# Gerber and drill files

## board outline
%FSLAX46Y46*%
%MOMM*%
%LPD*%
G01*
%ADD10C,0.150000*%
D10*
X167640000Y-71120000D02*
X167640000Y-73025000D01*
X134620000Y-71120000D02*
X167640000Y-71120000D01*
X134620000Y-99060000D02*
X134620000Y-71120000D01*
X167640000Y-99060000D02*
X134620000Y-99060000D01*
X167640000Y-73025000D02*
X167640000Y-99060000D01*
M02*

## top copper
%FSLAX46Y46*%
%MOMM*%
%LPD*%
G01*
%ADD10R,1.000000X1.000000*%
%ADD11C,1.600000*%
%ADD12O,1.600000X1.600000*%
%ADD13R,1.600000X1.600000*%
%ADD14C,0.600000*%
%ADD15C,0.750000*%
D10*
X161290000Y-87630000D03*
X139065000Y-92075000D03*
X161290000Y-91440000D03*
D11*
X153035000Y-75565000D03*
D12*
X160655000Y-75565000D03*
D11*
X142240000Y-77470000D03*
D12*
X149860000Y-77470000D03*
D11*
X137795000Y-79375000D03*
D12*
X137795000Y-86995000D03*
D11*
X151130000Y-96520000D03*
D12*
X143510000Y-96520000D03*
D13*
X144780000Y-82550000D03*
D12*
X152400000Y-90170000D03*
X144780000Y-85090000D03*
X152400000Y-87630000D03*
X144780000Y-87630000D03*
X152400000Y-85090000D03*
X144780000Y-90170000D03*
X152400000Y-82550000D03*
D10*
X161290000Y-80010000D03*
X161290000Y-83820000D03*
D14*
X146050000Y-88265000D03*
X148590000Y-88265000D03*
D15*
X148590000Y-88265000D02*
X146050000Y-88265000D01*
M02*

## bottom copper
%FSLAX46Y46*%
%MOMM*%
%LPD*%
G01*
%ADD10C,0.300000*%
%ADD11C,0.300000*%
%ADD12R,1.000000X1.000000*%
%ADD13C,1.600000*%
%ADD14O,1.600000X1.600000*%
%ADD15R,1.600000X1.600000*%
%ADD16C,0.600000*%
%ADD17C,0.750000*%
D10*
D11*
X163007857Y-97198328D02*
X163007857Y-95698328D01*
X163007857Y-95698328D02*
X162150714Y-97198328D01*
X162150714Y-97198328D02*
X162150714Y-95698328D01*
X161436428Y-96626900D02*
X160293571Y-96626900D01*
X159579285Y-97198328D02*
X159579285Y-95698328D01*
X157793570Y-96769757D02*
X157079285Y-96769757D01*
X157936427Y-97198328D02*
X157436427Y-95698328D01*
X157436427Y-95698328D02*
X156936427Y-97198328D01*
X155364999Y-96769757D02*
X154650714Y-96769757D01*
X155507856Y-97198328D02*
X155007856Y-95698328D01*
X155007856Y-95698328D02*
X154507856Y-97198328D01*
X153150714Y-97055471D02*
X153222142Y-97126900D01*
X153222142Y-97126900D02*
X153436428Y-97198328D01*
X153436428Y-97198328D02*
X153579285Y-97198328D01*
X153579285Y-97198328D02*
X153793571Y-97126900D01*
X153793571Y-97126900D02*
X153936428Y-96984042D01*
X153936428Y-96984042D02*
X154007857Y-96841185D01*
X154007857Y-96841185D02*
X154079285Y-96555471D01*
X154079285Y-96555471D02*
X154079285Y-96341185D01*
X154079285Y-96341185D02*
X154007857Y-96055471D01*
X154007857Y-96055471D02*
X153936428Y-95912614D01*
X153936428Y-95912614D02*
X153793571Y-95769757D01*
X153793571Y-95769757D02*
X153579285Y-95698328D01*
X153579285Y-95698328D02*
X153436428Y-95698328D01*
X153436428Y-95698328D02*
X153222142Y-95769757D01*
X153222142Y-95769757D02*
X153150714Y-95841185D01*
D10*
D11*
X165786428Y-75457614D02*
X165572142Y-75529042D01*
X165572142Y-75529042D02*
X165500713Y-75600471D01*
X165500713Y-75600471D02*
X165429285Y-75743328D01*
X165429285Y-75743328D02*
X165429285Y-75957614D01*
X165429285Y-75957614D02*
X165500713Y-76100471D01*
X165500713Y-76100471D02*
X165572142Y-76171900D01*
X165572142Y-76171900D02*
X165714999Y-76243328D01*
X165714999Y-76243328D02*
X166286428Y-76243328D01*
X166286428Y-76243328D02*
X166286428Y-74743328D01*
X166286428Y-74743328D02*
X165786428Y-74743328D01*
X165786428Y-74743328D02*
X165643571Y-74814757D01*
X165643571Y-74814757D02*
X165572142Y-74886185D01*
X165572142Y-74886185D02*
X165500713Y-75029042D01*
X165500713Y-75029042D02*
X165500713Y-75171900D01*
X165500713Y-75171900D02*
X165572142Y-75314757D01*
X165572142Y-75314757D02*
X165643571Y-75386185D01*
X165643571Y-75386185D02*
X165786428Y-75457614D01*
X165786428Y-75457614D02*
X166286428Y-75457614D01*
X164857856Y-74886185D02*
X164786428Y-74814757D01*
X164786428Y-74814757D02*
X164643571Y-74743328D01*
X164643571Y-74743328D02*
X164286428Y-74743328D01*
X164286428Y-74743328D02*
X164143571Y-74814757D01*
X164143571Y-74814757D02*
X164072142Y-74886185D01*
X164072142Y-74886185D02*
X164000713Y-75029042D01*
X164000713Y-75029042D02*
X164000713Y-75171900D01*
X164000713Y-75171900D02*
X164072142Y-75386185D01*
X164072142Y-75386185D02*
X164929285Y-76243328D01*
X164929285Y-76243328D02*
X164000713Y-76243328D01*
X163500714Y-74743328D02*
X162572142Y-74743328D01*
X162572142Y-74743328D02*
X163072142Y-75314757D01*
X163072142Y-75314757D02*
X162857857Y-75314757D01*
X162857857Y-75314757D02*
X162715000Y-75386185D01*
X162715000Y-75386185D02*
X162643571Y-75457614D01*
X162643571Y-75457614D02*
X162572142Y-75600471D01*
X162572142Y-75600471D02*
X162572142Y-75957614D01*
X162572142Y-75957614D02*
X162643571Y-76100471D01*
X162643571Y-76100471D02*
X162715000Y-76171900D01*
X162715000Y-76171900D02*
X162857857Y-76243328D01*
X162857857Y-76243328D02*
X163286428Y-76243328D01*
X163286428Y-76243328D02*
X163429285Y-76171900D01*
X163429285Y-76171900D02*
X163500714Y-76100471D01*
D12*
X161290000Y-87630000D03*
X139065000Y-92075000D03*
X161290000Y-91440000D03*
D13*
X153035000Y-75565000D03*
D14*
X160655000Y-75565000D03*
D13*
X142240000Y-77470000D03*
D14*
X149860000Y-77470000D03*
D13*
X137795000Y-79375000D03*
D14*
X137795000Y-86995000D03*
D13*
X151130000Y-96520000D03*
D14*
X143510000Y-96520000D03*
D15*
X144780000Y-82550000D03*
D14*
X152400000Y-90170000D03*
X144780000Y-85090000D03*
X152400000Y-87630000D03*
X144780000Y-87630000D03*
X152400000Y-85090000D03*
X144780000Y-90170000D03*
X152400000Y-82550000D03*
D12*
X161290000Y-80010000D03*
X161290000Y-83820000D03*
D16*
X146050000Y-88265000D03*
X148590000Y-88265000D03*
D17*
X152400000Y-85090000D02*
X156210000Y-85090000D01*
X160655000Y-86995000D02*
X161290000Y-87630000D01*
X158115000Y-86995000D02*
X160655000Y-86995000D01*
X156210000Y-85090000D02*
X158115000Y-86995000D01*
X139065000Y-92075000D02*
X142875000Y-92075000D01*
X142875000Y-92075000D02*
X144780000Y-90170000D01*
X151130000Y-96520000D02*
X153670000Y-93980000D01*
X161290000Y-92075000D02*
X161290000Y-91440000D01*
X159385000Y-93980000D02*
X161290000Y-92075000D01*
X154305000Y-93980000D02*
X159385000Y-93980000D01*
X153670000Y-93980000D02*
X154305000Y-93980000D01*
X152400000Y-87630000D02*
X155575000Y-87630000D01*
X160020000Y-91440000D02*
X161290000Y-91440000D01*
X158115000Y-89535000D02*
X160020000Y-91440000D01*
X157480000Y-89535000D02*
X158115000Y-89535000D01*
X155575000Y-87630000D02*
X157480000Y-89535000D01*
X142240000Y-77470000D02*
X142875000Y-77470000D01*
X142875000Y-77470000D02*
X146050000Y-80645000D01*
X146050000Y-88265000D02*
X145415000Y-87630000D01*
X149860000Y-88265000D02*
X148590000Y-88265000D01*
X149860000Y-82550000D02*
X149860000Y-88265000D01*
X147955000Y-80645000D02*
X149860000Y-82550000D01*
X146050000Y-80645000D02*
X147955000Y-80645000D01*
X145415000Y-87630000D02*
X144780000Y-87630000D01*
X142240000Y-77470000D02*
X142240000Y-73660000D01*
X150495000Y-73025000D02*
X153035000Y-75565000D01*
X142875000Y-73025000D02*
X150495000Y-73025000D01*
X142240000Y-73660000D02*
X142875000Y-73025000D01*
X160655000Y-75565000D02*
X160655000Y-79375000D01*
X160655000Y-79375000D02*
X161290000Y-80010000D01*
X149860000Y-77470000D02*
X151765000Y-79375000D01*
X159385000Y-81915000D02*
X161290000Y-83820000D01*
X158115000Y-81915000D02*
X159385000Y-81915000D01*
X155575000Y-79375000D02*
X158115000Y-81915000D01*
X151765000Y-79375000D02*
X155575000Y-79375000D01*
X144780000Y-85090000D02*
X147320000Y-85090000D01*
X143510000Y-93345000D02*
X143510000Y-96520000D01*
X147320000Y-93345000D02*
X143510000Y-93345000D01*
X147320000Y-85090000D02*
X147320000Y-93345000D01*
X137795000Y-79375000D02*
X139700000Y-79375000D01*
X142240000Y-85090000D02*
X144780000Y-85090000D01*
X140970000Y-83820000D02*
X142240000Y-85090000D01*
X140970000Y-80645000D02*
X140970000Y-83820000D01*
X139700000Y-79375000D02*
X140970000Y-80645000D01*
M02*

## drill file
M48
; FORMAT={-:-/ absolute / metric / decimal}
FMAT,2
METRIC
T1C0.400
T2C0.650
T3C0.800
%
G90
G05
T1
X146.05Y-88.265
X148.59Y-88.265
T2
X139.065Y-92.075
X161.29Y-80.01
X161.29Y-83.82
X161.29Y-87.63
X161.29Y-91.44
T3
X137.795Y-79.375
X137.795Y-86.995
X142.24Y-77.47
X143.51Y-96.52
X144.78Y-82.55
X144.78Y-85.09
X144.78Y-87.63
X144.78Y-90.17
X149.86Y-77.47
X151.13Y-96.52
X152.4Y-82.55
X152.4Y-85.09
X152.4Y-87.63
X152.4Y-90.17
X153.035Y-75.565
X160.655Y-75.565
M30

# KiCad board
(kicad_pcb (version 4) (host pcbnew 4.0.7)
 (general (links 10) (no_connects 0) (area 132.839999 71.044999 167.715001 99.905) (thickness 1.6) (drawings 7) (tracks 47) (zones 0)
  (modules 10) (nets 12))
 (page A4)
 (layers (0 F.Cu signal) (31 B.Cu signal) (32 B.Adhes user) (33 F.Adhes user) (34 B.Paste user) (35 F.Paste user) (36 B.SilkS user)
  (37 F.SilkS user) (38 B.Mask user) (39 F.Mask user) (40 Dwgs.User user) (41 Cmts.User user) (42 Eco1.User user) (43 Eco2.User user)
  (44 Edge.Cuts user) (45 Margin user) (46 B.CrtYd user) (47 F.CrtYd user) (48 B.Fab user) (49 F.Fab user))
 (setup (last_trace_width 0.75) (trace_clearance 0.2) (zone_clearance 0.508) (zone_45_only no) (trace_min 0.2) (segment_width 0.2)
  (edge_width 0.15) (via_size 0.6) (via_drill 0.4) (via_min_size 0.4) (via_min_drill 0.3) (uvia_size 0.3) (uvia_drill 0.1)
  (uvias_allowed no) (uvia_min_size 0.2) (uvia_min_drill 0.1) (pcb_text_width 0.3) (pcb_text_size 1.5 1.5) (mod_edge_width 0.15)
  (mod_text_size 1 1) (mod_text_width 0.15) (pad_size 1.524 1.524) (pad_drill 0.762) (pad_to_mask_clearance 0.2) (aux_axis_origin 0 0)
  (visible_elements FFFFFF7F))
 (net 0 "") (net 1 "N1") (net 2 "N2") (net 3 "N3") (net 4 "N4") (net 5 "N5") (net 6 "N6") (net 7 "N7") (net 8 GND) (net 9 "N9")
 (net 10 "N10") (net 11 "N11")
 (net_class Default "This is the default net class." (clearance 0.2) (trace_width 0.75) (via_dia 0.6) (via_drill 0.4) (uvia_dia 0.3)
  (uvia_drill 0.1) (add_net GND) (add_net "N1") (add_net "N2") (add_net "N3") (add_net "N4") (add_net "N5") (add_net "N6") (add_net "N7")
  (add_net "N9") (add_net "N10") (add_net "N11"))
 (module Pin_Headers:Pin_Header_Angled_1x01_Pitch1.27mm (layer F.Cu) (at 161.29 87.63)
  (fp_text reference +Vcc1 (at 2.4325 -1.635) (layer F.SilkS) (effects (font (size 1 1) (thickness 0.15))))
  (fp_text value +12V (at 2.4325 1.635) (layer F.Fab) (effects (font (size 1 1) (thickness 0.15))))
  (pad 1 thru_hole rect (at 0 0) (size 1 1) (drill 0.65) (layers *.Cu *.Mask) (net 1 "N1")))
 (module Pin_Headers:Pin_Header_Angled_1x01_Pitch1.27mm (layer F.Cu) (at 139.065 92.075 180)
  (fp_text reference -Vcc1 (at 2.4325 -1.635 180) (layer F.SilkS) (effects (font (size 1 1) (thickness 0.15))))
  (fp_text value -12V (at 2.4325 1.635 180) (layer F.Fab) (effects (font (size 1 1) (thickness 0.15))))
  (pad 1 thru_hole rect (at 0 0 180) (size 1 1) (drill 0.65) (layers *.Cu *.Mask) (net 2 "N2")))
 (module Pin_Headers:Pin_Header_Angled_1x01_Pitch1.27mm (layer F.Cu) (at 161.29 91.44)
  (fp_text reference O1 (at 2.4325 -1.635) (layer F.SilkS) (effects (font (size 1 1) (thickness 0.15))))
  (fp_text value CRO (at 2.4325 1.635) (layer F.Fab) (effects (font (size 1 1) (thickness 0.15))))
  (pad 1 thru_hole rect (at 0 0) (size 1 1) (drill 0.65) (layers *.Cu *.Mask) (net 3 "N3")))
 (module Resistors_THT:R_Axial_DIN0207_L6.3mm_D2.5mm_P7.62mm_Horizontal (layer F.Cu) (at 153.035 75.565)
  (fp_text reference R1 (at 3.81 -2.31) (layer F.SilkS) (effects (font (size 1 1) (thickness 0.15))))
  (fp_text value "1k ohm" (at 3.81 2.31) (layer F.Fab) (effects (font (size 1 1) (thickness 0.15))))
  (pad 1 thru_hole circle (at 0 0) (size 1.6 1.6) (drill 0.8) (layers *.Cu *.Mask) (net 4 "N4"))
  (pad 2 thru_hole oval (at 7.62 0) (size 1.6 1.6) (drill 0.8) (layers *.Cu *.Mask) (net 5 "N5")))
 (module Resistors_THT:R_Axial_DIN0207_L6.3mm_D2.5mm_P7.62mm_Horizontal (layer F.Cu) (at 142.24 77.47)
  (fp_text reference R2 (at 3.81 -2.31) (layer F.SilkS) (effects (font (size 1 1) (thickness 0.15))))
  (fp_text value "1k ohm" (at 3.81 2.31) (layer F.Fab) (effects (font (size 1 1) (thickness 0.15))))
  (pad 1 thru_hole circle (at 0 0) (size 1.6 1.6) (drill 0.8) (layers *.Cu *.Mask) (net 4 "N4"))
  (pad 2 thru_hole oval (at 7.62 0) (size 1.6 1.6) (drill 0.8) (layers *.Cu *.Mask) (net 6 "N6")))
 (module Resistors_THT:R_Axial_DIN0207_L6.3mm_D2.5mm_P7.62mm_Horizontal (layer F.Cu) (at 137.795 79.375 270)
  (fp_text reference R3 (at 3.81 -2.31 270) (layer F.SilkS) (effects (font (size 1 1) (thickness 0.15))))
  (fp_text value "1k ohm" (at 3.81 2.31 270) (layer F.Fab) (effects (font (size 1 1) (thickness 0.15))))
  (pad 1 thru_hole circle (at 0 0 270) (size 1.6 1.6) (drill 0.8) (layers *.Cu *.Mask) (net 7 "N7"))
  (pad 2 thru_hole oval (at 7.62 0 270) (size 1.6 1.6) (drill 0.8) (layers *.Cu *.Mask) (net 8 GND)))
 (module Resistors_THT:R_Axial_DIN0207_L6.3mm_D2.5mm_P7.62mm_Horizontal (layer F.Cu) (at 151.13 96.52 180)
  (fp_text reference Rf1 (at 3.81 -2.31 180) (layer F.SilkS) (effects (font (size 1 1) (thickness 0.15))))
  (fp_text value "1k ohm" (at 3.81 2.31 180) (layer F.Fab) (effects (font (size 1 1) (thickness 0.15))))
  (pad 1 thru_hole circle (at 0 0 180) (size 1.6 1.6) (drill 0.8) (layers *.Cu *.Mask) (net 3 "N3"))
  (pad 2 thru_hole oval (at 7.62 0 180) (size 1.6 1.6) (drill 0.8) (layers *.Cu *.Mask) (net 7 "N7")))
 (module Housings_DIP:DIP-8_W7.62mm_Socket (layer F.Cu) (at 144.78 82.55)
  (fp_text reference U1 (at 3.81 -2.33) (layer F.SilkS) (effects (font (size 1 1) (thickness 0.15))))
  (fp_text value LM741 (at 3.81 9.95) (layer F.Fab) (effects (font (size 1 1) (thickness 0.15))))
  (pad 1 thru_hole rect (at 0 0) (size 1.6 1.6) (drill 0.8) (layers *.Cu *.Mask) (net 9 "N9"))
  (pad 5 thru_hole oval (at 7.62 7.62) (size 1.6 1.6) (drill 0.8) (layers *.Cu *.Mask) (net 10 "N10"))
  (pad 2 thru_hole oval (at 0 2.54) (size 1.6 1.6) (drill 0.8) (layers *.Cu *.Mask) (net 7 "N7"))
  (pad 6 thru_hole oval (at 7.62 5.08) (size 1.6 1.6) (drill 0.8) (layers *.Cu *.Mask) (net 3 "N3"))
  (pad 3 thru_hole oval (at 0 5.08) (size 1.6 1.6) (drill 0.8) (layers *.Cu *.Mask) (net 4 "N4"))
  (pad 7 thru_hole oval (at 7.62 2.54) (size 1.6 1.6) (drill 0.8) (layers *.Cu *.Mask) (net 1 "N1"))
  (pad 4 thru_hole oval (at 0 7.62) (size 1.6 1.6) (drill 0.8) (layers *.Cu *.Mask) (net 2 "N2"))
  (pad 8 thru_hole oval (at 7.62 0) (size 1.6 1.6) (drill 0.8) (layers *.Cu *.Mask) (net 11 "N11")))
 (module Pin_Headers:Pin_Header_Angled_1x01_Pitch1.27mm (layer F.Cu) (at 161.29 80.01)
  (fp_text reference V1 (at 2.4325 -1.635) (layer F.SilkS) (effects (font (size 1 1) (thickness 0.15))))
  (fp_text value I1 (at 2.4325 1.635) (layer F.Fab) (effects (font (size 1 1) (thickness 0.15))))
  (pad 1 thru_hole rect (at 0 0) (size 1 1) (drill 0.65) (layers *.Cu *.Mask) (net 5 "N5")))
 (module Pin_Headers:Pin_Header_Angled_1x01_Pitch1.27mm (layer F.Cu) (at 161.29 83.82)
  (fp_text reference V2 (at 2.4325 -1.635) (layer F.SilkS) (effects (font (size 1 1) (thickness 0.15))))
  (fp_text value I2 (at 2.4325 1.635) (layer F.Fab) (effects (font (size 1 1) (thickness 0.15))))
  (pad 1 thru_hole rect (at 0 0) (size 1 1) (drill 0.65) (layers *.Cu *.Mask) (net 6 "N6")))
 (gr_line (start 167.64 71.12) (end 167.64 73.025) (angle 90) (layer Edge.Cuts) (width 0.15))
 (gr_line (start 134.62 71.12) (end 167.64 71.12) (angle 90) (layer Edge.Cuts) (width 0.15))
 (gr_line (start 134.62 99.06) (end 134.62 71.12) (angle 90) (layer Edge.Cuts) (width 0.15))
 (gr_line (start 167.64 99.06) (end 134.62 99.06) (angle 90) (layer Edge.Cuts) (width 0.15))
 (gr_line (start 167.64 73.025) (end 167.64 99.06) (angle 90) (layer Edge.Cuts) (width 0.15))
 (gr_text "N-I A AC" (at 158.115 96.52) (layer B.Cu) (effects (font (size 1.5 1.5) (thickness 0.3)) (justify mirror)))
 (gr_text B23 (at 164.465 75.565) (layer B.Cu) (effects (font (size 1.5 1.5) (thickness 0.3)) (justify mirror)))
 (segment (start 152.4 85.09) (end 156.21 85.09) (width 0.75) (layer B.Cu) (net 1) (status 400000))
 (segment (start 160.655 86.995) (end 161.29 87.63) (width 0.75) (layer B.Cu) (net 1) (status 800000))
 (segment (start 158.115 86.995) (end 160.655 86.995) (width 0.75) (layer B.Cu) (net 1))
 (segment (start 156.21 85.09) (end 158.115 86.995) (width 0.75) (layer B.Cu) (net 1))
 (segment (start 139.065 92.075) (end 142.875 92.075) (width 0.75) (layer B.Cu) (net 2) (status 400000))
 (segment (start 142.875 92.075) (end 144.78 90.17) (width 0.75) (layer B.Cu) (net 2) (status 800000))
 (segment (start 151.13 96.52) (end 153.67 93.98) (width 0.75) (layer B.Cu) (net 3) (status 400000))
 (segment (start 161.29 92.075) (end 161.29 91.44) (width 0.75) (layer B.Cu) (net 3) (status 800000))
 (segment (start 159.385 93.98) (end 161.29 92.075) (width 0.75) (layer B.Cu) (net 3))
 (segment (start 154.305 93.98) (end 159.385 93.98) (width 0.75) (layer B.Cu) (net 3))
 (segment (start 153.67 93.98) (end 154.305 93.98) (width 0.75) (layer B.Cu) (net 3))
 (segment (start 152.4 87.63) (end 155.575 87.63) (width 0.75) (layer B.Cu) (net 3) (status 400000))
 (segment (start 160.02 91.44) (end 161.29 91.44) (width 0.75) (layer B.Cu) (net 3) (status 800000))
 (segment (start 158.115 89.535) (end 160.02 91.44) (width 0.75) (layer B.Cu) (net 3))
 (segment (start 157.48 89.535) (end 158.115 89.535) (width 0.75) (layer B.Cu) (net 3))
 (segment (start 155.575 87.63) (end 157.48 89.535) (width 0.75) (layer B.Cu) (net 3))
 (segment (start 142.24 77.47) (end 142.875 77.47) (width 0.75) (layer B.Cu) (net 4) (status C00000))
 (segment (start 142.875 77.47) (end 146.05 80.645) (width 0.75) (layer B.Cu) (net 4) (status 400000))
 (segment (start 146.05 88.265) (end 145.415 87.63) (width 0.75) (layer B.Cu) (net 4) (status 800000))
 (via (at 146.05 88.265) (size 0.6) (drill 0.4) (layers F.Cu B.Cu) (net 4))
 (segment (start 148.59 88.265) (end 146.05 88.265) (width 0.75) (layer F.Cu) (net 4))
 (via (at 148.59 88.265) (size 0.6) (drill 0.4) (layers F.Cu B.Cu) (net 4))
 (segment (start 149.86 88.265) (end 148.59 88.265) (width 0.75) (layer B.Cu) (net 4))
 (segment (start 149.86 82.55) (end 149.86 88.265) (width 0.75) (layer B.Cu) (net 4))
 (segment (start 147.955 80.645) (end 149.86 82.55) (width 0.75) (layer B.Cu) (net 4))
 (segment (start 146.05 80.645) (end 147.955 80.645) (width 0.75) (layer B.Cu) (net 4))
 (segment (start 145.415 87.63) (end 144.78 87.63) (width 0.75) (layer B.Cu) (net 4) (status C00000))
 (segment (start 142.24 77.47) (end 142.24 73.66) (width 0.75) (layer B.Cu) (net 4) (status 400000))
 (segment (start 150.495 73.025) (end 153.035 75.565) (width 0.75) (layer B.Cu) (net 4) (status 800000))
 (segment (start 142.875 73.025) (end 150.495 73.025) (width 0.75) (layer B.Cu) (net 4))
 (segment (start 142.24 73.66) (end 142.875 73.025) (width 0.75) (layer B.Cu) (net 4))
 (segment (start 160.655 75.565) (end 160.655 79.375) (width 0.75) (layer B.Cu) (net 5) (status 400000))
 (segment (start 160.655 79.375) (end 161.29 80.01) (width 0.75) (layer B.Cu) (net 5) (status 800000))
 (segment (start 149.86 77.47) (end 151.765 79.375) (width 0.75) (layer B.Cu) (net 6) (status 400000))
 (segment (start 159.385 81.915) (end 161.29 83.82) (width 0.75) (layer B.Cu) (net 6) (status 800000))
 (segment (start 158.115 81.915) (end 159.385 81.915) (width 0.75) (layer B.Cu) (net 6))
 (segment (start 155.575 79.375) (end 158.115 81.915) (width 0.75) (layer B.Cu) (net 6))
 (segment (start 151.765 79.375) (end 155.575 79.375) (width 0.75) (layer B.Cu) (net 6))
 (segment (start 144.78 85.09) (end 147.32 85.09) (width 0.75) (layer B.Cu) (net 7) (status 400000))
 (segment (start 143.51 93.345) (end 143.51 96.52) (width 0.75) (layer B.Cu) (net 7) (status 800000))
 (segment (start 147.32 93.345) (end 143.51 93.345) (width 0.75) (layer B.Cu) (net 7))
 (segment (start 147.32 85.09) (end 147.32 93.345) (width 0.75) (layer B.Cu) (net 7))
 (segment (start 137.795 79.375) (end 139.7 79.375) (width 0.75) (layer B.Cu) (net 7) (status 400000))
 (segment (start 142.24 85.09) (end 144.78 85.09) (width 0.75) (layer B.Cu) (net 7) (status 800000))
 (segment (start 140.97 83.82) (end 142.24 85.09) (width 0.75) (layer B.Cu) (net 7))
 (segment (start 140.97 80.645) (end 140.97 83.82) (width 0.75) (layer B.Cu) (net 7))
 (segment (start 139.7 79.375) (end 140.97 80.645) (width 0.75) (layer B.Cu) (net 7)))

